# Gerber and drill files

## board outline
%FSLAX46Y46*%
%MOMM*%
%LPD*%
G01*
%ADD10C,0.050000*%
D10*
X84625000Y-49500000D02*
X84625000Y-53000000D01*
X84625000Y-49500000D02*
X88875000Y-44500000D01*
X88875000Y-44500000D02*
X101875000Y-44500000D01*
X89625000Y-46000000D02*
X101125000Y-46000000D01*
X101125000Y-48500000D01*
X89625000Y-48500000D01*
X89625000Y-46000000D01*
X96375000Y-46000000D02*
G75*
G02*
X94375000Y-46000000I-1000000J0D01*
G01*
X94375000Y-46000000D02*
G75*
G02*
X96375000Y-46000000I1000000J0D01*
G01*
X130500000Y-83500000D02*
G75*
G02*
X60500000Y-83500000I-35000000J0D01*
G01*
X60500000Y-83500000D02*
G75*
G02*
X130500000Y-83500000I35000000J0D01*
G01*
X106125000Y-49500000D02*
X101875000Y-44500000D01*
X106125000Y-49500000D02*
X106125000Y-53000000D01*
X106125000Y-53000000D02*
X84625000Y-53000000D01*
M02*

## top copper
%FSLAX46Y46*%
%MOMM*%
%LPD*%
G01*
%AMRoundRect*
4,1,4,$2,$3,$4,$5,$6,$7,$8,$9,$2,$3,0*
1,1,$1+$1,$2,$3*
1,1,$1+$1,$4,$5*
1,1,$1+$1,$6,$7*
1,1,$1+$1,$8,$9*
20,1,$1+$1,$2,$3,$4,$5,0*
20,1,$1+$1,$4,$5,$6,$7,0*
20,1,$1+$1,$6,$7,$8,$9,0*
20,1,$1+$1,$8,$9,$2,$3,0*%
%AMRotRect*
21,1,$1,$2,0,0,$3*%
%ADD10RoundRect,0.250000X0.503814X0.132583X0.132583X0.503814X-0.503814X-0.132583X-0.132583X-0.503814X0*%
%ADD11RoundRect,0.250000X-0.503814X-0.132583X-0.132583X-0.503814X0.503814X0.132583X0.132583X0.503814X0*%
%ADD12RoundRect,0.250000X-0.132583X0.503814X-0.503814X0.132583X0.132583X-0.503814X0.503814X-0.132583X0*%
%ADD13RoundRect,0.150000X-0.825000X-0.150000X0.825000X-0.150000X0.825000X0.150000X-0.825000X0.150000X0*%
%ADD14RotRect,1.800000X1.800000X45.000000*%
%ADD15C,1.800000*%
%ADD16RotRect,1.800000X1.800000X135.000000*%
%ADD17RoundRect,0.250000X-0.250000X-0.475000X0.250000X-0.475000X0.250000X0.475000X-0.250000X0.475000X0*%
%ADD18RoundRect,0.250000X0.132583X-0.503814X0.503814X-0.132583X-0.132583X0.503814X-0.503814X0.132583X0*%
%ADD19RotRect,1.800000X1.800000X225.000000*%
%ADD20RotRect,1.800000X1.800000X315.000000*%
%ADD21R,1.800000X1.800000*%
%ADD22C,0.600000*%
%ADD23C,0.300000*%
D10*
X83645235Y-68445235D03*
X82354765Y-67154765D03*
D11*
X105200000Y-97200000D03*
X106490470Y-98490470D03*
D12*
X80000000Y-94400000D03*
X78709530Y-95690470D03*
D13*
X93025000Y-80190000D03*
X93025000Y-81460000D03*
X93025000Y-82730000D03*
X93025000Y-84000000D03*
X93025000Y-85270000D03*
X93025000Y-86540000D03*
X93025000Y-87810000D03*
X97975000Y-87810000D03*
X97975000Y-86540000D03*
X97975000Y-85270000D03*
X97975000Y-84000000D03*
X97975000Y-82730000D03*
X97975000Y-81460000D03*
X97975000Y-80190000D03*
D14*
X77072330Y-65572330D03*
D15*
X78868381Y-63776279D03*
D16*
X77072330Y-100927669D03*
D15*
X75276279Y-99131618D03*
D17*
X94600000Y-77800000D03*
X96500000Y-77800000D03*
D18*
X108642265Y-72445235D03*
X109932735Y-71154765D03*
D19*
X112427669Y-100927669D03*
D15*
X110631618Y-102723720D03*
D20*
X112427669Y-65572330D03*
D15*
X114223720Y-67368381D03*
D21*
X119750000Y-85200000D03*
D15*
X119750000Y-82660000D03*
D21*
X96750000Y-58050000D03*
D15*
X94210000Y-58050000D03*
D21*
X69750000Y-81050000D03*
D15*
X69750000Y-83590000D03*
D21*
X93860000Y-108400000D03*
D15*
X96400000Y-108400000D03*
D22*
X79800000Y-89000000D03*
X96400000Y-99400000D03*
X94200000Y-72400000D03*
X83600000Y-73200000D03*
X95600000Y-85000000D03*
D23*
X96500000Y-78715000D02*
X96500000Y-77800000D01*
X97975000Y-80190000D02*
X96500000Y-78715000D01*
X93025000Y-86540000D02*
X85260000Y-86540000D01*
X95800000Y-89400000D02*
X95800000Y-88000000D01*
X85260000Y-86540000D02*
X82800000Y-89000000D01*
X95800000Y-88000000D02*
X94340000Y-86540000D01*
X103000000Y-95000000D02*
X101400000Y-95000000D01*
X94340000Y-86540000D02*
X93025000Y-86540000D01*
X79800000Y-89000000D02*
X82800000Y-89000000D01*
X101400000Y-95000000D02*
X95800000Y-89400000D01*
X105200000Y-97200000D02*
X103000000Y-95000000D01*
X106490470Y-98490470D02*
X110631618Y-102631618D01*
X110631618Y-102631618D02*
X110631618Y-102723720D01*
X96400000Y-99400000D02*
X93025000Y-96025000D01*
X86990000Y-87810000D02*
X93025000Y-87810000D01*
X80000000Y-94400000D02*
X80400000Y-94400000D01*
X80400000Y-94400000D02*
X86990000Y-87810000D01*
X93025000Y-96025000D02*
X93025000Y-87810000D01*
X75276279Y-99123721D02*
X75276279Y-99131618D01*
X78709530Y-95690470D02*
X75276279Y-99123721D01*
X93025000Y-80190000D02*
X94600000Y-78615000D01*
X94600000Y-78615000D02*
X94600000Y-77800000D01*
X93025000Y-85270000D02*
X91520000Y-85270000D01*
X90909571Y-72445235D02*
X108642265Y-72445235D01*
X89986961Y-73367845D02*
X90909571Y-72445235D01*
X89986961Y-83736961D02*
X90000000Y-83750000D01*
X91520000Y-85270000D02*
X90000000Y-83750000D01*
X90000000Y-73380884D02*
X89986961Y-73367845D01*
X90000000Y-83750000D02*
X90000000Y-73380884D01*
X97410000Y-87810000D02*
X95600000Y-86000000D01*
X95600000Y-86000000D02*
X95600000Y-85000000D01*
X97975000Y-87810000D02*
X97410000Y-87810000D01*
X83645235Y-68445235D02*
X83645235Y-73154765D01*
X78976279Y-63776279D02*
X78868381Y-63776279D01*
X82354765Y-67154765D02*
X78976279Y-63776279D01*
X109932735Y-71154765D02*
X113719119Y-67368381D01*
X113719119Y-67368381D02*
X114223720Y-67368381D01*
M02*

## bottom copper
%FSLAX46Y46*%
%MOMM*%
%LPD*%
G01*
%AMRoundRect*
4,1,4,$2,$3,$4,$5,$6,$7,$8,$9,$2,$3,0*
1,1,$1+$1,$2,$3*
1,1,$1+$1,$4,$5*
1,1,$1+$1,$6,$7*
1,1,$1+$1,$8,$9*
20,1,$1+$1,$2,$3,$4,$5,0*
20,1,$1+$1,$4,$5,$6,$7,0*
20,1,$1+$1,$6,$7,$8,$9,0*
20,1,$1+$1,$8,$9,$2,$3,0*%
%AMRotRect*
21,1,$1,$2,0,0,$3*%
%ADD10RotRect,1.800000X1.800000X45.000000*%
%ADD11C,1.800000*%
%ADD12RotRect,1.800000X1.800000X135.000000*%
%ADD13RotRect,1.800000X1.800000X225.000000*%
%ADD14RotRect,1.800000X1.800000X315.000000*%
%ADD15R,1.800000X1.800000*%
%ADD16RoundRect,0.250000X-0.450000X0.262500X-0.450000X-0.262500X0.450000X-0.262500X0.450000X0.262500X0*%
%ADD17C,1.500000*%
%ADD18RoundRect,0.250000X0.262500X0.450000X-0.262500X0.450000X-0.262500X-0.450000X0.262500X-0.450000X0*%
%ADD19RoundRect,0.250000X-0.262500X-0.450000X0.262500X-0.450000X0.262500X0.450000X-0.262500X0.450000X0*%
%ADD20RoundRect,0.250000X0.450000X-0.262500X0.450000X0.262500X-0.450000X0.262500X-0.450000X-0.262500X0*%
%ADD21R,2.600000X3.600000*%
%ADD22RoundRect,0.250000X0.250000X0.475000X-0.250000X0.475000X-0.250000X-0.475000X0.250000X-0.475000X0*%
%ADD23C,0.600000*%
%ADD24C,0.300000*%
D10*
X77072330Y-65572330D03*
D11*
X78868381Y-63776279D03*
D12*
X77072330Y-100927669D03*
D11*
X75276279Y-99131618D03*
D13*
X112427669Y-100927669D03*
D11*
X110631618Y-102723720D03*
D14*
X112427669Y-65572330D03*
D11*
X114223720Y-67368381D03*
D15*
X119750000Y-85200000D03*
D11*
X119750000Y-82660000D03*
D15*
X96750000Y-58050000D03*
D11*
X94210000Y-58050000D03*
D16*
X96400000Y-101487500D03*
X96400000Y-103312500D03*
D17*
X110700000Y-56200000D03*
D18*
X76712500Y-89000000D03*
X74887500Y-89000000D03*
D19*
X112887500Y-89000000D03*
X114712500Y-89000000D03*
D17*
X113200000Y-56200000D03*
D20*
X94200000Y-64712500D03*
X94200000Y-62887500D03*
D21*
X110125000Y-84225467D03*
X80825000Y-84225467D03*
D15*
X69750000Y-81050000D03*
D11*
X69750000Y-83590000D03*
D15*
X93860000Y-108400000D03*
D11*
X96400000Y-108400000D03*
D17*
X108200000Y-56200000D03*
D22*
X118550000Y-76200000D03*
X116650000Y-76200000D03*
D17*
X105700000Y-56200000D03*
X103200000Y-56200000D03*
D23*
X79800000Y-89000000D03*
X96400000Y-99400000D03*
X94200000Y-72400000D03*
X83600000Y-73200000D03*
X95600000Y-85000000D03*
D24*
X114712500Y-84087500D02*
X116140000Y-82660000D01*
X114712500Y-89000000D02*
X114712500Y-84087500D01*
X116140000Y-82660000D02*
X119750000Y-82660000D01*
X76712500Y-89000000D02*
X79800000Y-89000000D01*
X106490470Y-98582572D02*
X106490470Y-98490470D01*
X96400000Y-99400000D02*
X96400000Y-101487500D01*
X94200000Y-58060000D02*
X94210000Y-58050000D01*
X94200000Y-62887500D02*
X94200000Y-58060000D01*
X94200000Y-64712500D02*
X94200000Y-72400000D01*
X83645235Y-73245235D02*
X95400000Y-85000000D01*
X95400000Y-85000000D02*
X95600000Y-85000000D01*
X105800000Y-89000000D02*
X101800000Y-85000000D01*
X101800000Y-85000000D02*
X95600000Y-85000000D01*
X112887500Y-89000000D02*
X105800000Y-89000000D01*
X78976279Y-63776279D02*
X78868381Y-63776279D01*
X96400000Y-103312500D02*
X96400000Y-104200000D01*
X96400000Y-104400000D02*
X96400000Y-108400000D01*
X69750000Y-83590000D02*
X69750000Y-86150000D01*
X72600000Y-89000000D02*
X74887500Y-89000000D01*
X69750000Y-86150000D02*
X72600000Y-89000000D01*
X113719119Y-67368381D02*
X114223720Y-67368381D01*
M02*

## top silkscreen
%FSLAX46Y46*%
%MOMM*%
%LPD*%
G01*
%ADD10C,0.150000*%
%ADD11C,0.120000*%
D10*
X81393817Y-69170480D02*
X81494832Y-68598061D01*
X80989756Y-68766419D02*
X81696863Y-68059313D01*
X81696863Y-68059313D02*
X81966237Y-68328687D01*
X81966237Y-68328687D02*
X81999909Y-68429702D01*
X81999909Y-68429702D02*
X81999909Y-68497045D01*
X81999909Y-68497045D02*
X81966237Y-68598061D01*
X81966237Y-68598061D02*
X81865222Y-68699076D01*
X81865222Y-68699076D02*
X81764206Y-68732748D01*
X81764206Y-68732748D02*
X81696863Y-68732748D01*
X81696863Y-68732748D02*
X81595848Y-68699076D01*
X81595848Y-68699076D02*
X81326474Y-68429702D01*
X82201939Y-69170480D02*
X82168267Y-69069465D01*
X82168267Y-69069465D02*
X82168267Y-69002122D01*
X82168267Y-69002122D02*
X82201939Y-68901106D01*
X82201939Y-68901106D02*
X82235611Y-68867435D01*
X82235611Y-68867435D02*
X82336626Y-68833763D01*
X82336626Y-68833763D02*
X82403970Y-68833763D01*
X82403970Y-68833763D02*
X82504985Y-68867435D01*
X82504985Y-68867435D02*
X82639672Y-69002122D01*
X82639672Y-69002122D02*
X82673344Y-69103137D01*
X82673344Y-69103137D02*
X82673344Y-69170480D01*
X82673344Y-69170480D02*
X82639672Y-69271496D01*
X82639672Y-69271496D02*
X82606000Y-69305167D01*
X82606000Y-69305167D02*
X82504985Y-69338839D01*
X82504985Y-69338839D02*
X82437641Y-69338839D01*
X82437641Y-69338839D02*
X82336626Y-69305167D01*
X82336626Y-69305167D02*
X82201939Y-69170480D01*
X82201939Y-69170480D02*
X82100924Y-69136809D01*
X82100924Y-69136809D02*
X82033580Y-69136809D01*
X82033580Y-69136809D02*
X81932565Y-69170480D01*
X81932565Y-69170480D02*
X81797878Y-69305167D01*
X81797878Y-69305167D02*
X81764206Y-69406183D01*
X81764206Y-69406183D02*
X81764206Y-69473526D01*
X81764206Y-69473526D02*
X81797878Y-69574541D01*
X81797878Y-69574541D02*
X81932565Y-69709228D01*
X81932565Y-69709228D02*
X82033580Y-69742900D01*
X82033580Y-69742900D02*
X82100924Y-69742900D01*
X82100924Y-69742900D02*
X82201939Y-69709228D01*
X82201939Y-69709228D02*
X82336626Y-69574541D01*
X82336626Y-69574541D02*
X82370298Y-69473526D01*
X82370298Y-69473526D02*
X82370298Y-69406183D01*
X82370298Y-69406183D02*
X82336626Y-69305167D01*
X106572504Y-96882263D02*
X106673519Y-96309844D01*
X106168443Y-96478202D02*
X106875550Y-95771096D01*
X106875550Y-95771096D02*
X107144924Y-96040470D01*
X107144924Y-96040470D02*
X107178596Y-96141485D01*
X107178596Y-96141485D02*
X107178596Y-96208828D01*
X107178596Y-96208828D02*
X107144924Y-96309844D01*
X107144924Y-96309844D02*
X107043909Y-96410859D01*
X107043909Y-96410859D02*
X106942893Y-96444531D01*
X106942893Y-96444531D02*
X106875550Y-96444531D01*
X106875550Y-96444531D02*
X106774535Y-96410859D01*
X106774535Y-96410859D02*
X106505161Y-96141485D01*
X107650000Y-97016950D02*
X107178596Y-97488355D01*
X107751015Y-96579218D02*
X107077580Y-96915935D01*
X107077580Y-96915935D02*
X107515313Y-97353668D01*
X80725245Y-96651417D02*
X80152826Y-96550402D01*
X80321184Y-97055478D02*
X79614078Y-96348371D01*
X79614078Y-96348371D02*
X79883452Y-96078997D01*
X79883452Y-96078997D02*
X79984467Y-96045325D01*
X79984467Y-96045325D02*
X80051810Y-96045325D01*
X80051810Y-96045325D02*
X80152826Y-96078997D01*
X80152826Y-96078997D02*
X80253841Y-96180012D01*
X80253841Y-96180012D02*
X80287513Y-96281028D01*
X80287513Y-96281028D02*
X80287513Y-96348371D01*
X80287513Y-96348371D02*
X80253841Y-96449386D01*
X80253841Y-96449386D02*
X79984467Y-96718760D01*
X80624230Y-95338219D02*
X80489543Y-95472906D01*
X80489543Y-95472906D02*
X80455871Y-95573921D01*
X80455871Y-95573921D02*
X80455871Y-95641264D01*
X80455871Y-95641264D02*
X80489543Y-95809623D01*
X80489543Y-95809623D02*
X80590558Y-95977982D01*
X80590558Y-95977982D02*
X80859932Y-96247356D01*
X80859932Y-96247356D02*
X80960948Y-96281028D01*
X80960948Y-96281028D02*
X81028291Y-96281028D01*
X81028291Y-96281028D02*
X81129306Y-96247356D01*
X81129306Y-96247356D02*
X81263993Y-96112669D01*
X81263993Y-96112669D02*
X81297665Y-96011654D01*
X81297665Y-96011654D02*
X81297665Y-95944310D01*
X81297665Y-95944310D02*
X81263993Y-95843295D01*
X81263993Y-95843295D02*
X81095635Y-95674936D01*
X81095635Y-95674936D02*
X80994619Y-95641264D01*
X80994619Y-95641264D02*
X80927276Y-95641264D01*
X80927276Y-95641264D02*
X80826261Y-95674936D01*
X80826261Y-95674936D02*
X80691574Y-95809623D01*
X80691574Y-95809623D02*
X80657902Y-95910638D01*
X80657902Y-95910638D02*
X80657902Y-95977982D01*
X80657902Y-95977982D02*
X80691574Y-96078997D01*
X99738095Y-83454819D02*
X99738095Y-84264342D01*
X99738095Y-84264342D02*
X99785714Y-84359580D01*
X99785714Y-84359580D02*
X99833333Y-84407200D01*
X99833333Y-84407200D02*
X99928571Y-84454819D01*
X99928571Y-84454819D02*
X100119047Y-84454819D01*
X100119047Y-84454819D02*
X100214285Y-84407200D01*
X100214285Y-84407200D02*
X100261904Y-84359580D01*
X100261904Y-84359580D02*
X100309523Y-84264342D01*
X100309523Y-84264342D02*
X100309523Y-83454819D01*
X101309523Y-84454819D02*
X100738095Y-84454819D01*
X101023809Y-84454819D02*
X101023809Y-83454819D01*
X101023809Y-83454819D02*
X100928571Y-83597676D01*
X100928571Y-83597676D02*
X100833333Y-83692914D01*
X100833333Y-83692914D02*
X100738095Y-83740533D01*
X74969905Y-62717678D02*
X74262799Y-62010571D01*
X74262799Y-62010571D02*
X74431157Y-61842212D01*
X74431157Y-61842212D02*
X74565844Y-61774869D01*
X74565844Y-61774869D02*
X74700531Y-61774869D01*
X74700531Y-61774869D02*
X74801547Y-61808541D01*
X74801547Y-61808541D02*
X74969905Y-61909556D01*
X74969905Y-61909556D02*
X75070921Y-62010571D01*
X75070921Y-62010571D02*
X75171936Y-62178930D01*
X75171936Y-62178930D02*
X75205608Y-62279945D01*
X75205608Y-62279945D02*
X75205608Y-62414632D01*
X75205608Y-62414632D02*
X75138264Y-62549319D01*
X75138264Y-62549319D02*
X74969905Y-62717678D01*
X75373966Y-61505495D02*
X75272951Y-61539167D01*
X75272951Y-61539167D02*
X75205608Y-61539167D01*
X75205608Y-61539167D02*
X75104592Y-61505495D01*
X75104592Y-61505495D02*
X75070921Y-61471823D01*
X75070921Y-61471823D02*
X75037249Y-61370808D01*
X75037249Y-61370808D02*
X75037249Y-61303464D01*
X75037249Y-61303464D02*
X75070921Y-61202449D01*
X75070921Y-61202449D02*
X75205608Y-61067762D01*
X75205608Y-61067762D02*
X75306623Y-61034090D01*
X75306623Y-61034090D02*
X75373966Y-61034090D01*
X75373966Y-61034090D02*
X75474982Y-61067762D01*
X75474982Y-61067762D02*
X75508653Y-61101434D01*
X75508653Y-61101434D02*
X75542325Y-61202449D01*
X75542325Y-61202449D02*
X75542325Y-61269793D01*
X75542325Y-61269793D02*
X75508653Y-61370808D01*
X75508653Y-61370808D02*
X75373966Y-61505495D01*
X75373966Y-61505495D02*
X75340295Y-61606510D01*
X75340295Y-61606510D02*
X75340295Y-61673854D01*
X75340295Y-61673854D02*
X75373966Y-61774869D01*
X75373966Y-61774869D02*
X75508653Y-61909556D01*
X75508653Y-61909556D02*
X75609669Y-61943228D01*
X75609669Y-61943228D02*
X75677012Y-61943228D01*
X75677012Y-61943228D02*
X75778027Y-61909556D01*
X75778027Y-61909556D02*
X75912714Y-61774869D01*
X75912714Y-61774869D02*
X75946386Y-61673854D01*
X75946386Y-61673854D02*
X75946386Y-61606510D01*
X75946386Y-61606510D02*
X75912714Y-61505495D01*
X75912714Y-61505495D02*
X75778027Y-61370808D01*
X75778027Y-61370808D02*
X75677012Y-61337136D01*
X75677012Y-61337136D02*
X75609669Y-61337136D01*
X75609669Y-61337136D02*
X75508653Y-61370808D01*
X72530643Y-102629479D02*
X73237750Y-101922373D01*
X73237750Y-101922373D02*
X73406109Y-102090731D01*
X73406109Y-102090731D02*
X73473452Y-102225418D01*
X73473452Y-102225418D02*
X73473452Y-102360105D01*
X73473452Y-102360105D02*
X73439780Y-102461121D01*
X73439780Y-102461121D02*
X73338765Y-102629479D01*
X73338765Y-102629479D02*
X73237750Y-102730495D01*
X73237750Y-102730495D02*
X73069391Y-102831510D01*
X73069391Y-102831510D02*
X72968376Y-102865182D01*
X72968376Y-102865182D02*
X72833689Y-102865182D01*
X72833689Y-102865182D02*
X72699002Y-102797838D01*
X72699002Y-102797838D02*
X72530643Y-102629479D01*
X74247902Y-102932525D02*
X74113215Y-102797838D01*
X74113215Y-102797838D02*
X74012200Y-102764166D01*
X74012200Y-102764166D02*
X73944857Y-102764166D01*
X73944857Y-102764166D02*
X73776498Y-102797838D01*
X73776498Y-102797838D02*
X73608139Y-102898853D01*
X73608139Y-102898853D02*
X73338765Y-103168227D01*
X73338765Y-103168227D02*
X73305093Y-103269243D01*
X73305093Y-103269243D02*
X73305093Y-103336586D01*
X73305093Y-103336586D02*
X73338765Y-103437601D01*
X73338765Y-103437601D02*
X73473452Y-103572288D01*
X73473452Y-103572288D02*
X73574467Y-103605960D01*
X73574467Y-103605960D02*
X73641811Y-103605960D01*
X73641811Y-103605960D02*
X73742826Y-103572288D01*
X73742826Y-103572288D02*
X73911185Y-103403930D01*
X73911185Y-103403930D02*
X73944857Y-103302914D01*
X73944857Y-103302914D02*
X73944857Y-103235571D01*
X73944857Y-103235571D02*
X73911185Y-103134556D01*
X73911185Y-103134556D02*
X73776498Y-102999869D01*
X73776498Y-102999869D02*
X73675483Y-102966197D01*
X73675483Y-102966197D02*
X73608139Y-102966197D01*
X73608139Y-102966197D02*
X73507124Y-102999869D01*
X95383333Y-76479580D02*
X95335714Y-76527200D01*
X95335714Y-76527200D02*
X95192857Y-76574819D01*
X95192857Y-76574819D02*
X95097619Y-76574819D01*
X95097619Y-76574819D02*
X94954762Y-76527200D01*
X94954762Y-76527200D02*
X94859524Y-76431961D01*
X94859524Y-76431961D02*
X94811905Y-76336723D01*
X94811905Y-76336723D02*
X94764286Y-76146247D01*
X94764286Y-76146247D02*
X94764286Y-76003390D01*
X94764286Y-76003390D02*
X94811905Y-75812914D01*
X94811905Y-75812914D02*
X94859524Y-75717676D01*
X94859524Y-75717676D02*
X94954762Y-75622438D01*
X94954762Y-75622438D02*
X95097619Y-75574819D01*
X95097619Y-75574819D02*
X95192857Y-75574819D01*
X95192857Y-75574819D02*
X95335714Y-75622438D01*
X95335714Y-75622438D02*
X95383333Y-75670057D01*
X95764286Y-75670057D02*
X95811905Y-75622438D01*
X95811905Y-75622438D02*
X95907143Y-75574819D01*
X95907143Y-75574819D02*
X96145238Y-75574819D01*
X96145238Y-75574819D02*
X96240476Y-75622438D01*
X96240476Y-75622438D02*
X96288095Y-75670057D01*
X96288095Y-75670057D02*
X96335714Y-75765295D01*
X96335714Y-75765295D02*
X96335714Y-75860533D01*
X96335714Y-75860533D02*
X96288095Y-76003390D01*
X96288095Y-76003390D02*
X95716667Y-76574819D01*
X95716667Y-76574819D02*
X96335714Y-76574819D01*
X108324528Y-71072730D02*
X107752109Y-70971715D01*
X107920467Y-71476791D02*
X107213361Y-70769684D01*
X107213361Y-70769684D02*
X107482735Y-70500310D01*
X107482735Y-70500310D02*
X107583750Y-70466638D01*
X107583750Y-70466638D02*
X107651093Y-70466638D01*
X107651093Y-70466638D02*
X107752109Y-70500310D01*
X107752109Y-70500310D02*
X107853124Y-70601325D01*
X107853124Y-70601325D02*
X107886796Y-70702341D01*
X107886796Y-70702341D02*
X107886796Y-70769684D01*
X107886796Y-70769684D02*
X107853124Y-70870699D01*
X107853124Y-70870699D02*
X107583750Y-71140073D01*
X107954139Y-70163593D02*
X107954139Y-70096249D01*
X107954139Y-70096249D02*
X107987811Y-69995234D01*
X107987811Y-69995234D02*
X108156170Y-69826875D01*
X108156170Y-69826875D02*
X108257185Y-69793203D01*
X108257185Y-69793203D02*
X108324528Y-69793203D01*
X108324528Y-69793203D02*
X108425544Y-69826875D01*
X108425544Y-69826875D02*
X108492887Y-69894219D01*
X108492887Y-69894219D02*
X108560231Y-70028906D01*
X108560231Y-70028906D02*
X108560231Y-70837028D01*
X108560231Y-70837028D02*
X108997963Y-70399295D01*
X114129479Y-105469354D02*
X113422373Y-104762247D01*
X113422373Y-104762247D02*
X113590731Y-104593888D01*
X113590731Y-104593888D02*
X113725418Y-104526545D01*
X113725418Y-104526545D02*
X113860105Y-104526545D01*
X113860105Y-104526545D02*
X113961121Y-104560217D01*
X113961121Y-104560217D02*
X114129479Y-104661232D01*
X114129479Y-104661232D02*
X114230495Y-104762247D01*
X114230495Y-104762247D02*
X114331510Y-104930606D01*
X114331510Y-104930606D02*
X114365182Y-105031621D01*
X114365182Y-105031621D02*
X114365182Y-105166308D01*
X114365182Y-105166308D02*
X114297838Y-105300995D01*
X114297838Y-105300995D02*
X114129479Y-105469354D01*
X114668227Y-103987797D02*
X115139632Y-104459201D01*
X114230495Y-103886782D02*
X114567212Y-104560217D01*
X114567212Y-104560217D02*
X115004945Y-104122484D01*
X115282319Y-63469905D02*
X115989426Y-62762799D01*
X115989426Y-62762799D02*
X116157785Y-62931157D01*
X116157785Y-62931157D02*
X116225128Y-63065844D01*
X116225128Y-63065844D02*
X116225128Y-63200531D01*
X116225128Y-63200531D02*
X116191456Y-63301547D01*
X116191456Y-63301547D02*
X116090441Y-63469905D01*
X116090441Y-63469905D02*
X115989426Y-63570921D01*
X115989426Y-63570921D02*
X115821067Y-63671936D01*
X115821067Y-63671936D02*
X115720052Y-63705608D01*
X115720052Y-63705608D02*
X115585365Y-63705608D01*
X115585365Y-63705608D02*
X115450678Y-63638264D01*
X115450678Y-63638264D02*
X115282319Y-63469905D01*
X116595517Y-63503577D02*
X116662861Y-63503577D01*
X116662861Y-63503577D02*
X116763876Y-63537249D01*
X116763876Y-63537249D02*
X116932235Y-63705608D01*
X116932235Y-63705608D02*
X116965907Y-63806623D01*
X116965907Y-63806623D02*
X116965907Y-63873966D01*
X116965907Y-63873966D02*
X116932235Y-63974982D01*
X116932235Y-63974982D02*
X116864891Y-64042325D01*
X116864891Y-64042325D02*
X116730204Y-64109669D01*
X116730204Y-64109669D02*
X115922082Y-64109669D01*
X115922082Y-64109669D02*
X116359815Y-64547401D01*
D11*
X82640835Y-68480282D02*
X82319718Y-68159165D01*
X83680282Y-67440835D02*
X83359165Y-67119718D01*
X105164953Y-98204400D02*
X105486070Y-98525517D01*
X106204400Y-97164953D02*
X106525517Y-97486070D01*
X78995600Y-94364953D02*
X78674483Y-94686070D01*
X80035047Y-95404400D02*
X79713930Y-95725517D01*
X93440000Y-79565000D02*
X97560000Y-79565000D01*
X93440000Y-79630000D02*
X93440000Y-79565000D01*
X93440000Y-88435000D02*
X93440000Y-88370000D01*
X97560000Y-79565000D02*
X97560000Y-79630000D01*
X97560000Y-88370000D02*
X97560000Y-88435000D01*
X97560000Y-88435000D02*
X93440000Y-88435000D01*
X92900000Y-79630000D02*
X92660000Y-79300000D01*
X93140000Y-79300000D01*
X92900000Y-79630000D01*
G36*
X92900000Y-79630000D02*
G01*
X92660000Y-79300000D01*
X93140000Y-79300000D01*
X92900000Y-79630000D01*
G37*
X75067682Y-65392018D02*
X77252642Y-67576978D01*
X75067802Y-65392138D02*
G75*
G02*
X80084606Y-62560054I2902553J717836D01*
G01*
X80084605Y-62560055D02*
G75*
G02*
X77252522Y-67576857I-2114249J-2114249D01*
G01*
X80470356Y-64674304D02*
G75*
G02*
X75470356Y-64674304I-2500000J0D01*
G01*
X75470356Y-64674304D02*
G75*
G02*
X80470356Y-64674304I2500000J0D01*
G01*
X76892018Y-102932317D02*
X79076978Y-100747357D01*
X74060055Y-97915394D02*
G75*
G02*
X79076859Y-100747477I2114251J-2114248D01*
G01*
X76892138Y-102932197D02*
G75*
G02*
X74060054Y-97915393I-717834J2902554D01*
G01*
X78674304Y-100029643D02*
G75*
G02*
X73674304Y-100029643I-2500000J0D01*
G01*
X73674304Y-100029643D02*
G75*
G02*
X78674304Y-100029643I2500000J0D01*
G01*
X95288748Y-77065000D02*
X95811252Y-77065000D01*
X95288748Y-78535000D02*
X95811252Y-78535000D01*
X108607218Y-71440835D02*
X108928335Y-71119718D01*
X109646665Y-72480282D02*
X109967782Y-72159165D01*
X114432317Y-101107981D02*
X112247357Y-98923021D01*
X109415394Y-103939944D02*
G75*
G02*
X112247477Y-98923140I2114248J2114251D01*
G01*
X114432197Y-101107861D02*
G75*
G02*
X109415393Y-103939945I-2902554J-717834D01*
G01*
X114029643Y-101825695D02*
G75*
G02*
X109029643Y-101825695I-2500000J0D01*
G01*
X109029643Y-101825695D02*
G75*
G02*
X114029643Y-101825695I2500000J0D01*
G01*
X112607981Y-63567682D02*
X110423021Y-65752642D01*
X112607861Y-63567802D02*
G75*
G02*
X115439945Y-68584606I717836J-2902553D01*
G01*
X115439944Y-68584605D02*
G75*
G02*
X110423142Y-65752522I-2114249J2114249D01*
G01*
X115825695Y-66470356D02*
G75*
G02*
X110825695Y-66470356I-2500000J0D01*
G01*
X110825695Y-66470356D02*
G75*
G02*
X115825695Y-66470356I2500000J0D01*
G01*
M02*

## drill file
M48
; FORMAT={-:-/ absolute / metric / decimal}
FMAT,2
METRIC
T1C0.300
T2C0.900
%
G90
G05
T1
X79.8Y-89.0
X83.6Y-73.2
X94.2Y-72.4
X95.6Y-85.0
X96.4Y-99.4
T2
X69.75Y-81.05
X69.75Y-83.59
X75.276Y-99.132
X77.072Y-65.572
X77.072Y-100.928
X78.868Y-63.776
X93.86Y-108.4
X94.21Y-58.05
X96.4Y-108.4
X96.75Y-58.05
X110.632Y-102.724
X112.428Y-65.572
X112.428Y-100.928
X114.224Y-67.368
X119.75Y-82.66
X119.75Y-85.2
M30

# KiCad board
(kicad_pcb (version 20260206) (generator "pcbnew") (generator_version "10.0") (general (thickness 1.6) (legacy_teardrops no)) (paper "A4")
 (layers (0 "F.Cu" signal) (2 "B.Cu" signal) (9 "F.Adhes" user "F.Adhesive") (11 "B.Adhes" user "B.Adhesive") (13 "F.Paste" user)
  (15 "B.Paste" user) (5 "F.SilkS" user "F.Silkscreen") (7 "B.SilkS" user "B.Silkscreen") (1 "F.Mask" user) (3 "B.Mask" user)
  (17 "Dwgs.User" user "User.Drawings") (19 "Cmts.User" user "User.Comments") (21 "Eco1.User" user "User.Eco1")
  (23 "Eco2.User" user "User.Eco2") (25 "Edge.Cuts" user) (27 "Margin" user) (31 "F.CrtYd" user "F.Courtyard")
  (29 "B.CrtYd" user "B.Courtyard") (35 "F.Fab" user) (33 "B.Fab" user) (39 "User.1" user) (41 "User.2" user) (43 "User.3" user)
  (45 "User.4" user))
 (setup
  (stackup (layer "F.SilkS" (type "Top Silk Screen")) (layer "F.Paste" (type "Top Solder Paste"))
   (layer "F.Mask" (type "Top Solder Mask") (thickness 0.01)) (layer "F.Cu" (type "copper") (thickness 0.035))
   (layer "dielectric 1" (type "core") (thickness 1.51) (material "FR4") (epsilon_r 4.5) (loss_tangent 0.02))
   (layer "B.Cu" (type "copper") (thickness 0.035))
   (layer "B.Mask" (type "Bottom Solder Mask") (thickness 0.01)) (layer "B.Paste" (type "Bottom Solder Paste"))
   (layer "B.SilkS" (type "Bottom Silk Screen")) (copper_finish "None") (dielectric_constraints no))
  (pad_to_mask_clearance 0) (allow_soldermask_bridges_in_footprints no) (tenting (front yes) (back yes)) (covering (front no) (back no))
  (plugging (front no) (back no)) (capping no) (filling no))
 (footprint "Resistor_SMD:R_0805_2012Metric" (layer "F.Cu") (at 83 67.8 135)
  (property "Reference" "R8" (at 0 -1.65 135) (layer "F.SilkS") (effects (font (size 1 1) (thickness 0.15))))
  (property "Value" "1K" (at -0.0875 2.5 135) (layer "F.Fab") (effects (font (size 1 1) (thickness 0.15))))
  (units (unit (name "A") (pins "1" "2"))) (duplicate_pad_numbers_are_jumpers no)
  (fp_line (start -0.227064 -0.735) (end 0.227064 -0.735) (stroke (width 0.12) (type solid)) (layer "F.SilkS"))
  (fp_line (start -0.227064 0.735) (end 0.227064 0.735) (stroke (width 0.12) (type solid)) (layer "F.SilkS"))
  (pad "1" smd roundrect (at -0.9125 0 135) (size 1.025 1.4) (layers "F.Cu" "F.Mask" "F.Paste") (roundrect_rratio 0.243902)
   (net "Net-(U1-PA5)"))
  (pad "2" smd roundrect (at 0.9125 0 135) (size 1.025 1.4) (layers "F.Cu" "F.Mask" "F.Paste") (roundrect_rratio 0.243902)
   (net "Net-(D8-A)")))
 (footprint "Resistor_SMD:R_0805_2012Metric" (layer "F.Cu") (at 105.845235 97.845235 -45)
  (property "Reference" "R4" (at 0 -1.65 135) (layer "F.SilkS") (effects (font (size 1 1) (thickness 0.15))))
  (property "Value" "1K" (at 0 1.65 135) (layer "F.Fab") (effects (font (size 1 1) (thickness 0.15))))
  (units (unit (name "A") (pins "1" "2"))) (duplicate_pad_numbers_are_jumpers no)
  (fp_line (start -0.227064 0.735) (end 0.227064 0.735) (stroke (width 0.12) (type solid)) (layer "F.SilkS"))
  (fp_line (start -0.227064 -0.735) (end 0.227064 -0.735) (stroke (width 0.12) (type solid)) (layer "F.SilkS"))
  (pad "1" smd roundrect (at -0.9125 0 315) (size 1.025 1.4) (layers "F.Cu" "F.Mask" "F.Paste") (roundrect_rratio 0.243902)
   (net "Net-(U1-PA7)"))
  (pad "2" smd roundrect (at 0.9125 0 315) (size 1.025 1.4) (layers "F.Cu" "F.Mask" "F.Paste") (roundrect_rratio 0.243902)
   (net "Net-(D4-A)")))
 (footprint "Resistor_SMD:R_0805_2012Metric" (layer "F.Cu") (at 79.354765 95.045235 -135)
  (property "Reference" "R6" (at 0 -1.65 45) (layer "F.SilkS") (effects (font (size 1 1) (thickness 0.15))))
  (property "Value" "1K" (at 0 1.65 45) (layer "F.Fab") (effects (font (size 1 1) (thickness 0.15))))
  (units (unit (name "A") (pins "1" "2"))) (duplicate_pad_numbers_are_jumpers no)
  (fp_line (start -0.227064 0.735) (end 0.227064 0.735) (stroke (width 0.12) (type solid)) (layer "F.SilkS"))
  (fp_line (start -0.227064 -0.735) (end 0.227064 -0.735) (stroke (width 0.12) (type solid)) (layer "F.SilkS"))
  (pad "1" smd roundrect (at -0.9125 0 225) (size 1.025 1.4) (layers "F.Cu" "F.Mask" "F.Paste") (roundrect_rratio 0.243902)
   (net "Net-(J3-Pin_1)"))
  (pad "2" smd roundrect (at 0.9125 0 225) (size 1.025 1.4) (layers "F.Cu" "F.Mask" "F.Paste") (roundrect_rratio 0.243902)
   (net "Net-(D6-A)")))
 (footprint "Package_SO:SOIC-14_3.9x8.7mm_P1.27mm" (layer "F.Cu") (at 95.5 84)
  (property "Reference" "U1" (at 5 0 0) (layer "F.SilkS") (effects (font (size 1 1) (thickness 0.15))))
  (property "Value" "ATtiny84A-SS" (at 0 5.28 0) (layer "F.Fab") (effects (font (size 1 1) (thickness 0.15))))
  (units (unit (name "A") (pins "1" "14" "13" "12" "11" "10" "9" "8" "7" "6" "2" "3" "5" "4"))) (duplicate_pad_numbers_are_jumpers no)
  (fp_line (start -2.06 -4.435) (end 2.06 -4.435) (stroke (width 0.12) (type solid)) (layer "F.SilkS"))
  (fp_line (start -2.06 -4.37) (end -2.06 -4.435) (stroke (width 0.12) (type solid)) (layer "F.SilkS"))
  (fp_line (start -2.06 4.435) (end -2.06 4.37) (stroke (width 0.12) (type solid)) (layer "F.SilkS"))
  (fp_line (start 2.06 -4.435) (end 2.06 -4.37) (stroke (width 0.12) (type solid)) (layer "F.SilkS"))
  (fp_line (start 2.06 4.37) (end 2.06 4.435) (stroke (width 0.12) (type solid)) (layer "F.SilkS"))
  (fp_line (start 2.06 4.435) (end -2.06 4.435) (stroke (width 0.12) (type solid)) (layer "F.SilkS"))
  (fp_poly (pts (xy -2.6 -4.37) (xy -2.84 -4.7) (xy -2.36 -4.7)) (stroke (width 0.12) (type solid)) (fill yes) (layer "F.SilkS"))
  (pad "1" smd roundrect (at -2.475 -3.81) (size 1.95 0.6) (layers "F.Cu" "F.Mask" "F.Paste") (roundrect_rratio 0.25) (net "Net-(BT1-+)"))
  (pad "2" smd roundrect (at -2.475 -2.54) (size 1.95 0.6) (layers "F.Cu" "F.Mask" "F.Paste") (roundrect_rratio 0.25)
   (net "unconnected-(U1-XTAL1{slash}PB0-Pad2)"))
  (pad "3" smd roundrect (at -2.475 -1.27) (size 1.95 0.6) (layers "F.Cu" "F.Mask" "F.Paste") (roundrect_rratio 0.25)
   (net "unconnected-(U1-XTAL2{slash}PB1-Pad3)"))
  (pad "4" smd roundrect (at -2.475 0) (size 1.95 0.6) (layers "F.Cu" "F.Mask" "F.Paste") (roundrect_rratio 0.25) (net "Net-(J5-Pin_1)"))
  (pad "5" smd roundrect (at -2.475 1.27) (size 1.95 0.6) (layers "F.Cu" "F.Mask" "F.Paste") (roundrect_rratio 0.25) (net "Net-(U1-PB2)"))
  (pad "6" smd roundrect (at -2.475 2.54) (size 1.95 0.6) (layers "F.Cu" "F.Mask" "F.Paste") (roundrect_rratio 0.25) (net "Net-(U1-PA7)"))
  (pad "7" smd roundrect (at -2.475 3.81) (size 1.95 0.6) (layers "F.Cu" "F.Mask" "F.Paste") (roundrect_rratio 0.25) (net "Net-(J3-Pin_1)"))
  (pad "8" smd roundrect (at 2.475 3.81) (size 1.95 0.6) (layers "F.Cu" "F.Mask" "F.Paste") (roundrect_rratio 0.25) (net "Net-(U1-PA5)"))
  (pad "9" smd roundrect (at 2.475 2.54) (size 1.95 0.6) (layers "F.Cu" "F.Mask" "F.Paste") (roundrect_rratio 0.25) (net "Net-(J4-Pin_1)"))
  (pad "10" smd roundrect (at 2.475 1.27) (size 1.95 0.6) (layers "F.Cu" "F.Mask" "F.Paste") (roundrect_rratio 0.25)
   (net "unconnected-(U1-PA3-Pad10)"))
  (pad "11" smd roundrect (at 2.475 0) (size 1.95 0.6) (layers "F.Cu" "F.Mask" "F.Paste") (roundrect_rratio 0.25)
   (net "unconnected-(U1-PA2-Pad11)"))
  (pad "12" smd roundrect (at 2.475 -1.27) (size 1.95 0.6) (layers "F.Cu" "F.Mask" "F.Paste") (roundrect_rratio 0.25) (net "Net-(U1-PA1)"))
  (pad "13" smd roundrect (at 2.475 -2.54) (size 1.95 0.6) (layers "F.Cu" "F.Mask" "F.Paste") (roundrect_rratio 0.25)
   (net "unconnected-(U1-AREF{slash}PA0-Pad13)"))
  (pad "14" smd roundrect (at 2.475 -3.81) (size 1.95 0.6) (layers "F.Cu" "F.Mask" "F.Paste") (roundrect_rratio 0.25) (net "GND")))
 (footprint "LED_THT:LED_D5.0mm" (layer "F.Cu") (at 77.07233 65.57233 45)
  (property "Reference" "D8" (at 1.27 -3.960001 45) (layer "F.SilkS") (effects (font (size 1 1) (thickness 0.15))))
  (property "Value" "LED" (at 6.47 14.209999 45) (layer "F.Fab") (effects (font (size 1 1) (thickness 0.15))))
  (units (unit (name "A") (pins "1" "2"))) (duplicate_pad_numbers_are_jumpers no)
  (fp_line (start -1.29 -1.545) (end -1.29 1.545) (stroke (width 0.12) (type solid)) (layer "F.SilkS"))
  (fp_arc (start -1.29 -1.54483) (mid 2.07178 -2.880496) (end 4.26 0) (stroke (width 0.12) (type solid)) (layer "F.SilkS"))
  (fp_arc (start 4.26 0) (mid 2.07178 2.880495) (end -1.29 1.54483) (stroke (width 0.12) (type solid)) (layer "F.SilkS"))
  (fp_circle (center 1.270001 0) (end 3.770001 0) (stroke (width 0.12) (type solid)) (fill no) (layer "F.SilkS"))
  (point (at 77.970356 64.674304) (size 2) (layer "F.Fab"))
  (pad "1" thru_hole rect (at 0 0 45) (size 1.8 1.8) (drill 0.9) (layers "*.Cu" "*.Mask") (remove_unused_layers no) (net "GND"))
  (pad "2" thru_hole circle (at 2.54 0 45) (size 1.8 1.8) (drill 0.9) (layers "*.Cu" "*.Mask") (remove_unused_layers no) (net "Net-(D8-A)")))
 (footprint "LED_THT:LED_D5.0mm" (layer "F.Cu") (at 77.07233 100.927669 135)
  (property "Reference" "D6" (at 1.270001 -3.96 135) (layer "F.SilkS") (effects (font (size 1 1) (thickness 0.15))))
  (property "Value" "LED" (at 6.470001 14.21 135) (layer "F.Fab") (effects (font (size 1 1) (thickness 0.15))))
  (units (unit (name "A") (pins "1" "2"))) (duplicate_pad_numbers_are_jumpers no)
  (fp_line (start -1.29 -1.545) (end -1.29 1.545) (stroke (width 0.12) (type solid)) (layer "F.SilkS"))
  (fp_arc (start 4.26 0) (mid 2.071779 2.880496) (end -1.29 1.54483) (stroke (width 0.12) (type solid)) (layer "F.SilkS"))
  (fp_arc (start -1.29 -1.54483) (mid 2.071779 -2.880496) (end 4.26 0) (stroke (width 0.12) (type solid)) (layer "F.SilkS"))
  (fp_circle (center 1.270001 0) (end 3.770001 0) (stroke (width 0.12) (type solid)) (fill no) (layer "F.SilkS"))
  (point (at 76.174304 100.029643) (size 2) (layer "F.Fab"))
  (pad "1" thru_hole rect (at 0 0 135) (size 1.8 1.8) (drill 0.9) (layers "*.Cu" "*.Mask") (remove_unused_layers no) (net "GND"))
  (pad "2" thru_hole circle (at 2.54 0 135) (size 1.8 1.8) (drill 0.9) (layers "*.Cu" "*.Mask") (remove_unused_layers no) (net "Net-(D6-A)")))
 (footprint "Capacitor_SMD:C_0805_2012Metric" (layer "F.Cu") (at 95.55 77.8)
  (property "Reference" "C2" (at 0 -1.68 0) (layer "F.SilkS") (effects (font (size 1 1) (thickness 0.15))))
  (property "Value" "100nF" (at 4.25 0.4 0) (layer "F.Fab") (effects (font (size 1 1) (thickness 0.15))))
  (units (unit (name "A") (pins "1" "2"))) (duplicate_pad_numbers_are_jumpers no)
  (fp_line (start -0.261252 -0.735) (end 0.261252 -0.735) (stroke (width 0.12) (type solid)) (layer "F.SilkS"))
  (fp_line (start -0.261252 0.735) (end 0.261252 0.735) (stroke (width 0.12) (type solid)) (layer "F.SilkS"))
  (pad "1" smd roundrect (at -0.95 0) (size 1 1.45) (layers "F.Cu" "F.Mask" "F.Paste") (roundrect_rratio 0.25) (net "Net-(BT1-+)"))
  (pad "2" smd roundrect (at 0.95 0) (size 1 1.45) (layers "F.Cu" "F.Mask" "F.Paste") (roundrect_rratio 0.25) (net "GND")))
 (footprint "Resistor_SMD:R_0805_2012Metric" (layer "F.Cu") (at 109.2875 71.8 45)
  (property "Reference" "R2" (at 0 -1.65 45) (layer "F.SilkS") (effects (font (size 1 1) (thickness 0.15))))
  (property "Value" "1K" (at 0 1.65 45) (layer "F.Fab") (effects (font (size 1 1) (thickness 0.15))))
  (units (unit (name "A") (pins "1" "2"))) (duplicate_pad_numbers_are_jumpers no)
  (fp_line (start -0.227064 -0.735) (end 0.227064 -0.735) (stroke (width 0.12) (type solid)) (layer "F.SilkS"))
  (fp_line (start -0.227064 0.735) (end 0.227064 0.735) (stroke (width 0.12) (type solid)) (layer "F.SilkS"))
  (pad "1" smd roundrect (at -0.9125 0 45) (size 1.025 1.4) (layers "F.Cu" "F.Mask" "F.Paste") (roundrect_rratio 0.243902)
   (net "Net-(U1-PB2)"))
  (pad "2" smd roundrect (at 0.9125 0 45) (size 1.025 1.4) (layers "F.Cu" "F.Mask" "F.Paste") (roundrect_rratio 0.243902) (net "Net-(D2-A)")))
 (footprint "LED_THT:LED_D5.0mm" (layer "F.Cu") (at 112.427669 100.927669 -135)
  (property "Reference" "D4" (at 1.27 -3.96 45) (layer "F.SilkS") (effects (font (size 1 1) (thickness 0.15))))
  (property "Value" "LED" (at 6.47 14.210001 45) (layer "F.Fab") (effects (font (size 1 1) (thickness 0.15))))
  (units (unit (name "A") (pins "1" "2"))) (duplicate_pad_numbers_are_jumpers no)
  (fp_line (start -1.29 -1.545) (end -1.29 1.545) (stroke (width 0.12) (type solid)) (layer "F.SilkS"))
  (fp_arc (start 4.26 0) (mid 2.071779 2.880496) (end -1.29 1.54483) (stroke (width 0.12) (type solid)) (layer "F.SilkS"))
  (fp_arc (start -1.29 -1.54483) (mid 2.071779 -2.880496) (end 4.26 0) (stroke (width 0.12) (type solid)) (layer "F.SilkS"))
  (fp_circle (center 1.270001 0) (end 3.770001 0) (stroke (width 0.12) (type solid)) (fill no) (layer "F.SilkS"))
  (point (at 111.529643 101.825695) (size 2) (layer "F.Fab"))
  (pad "1" thru_hole rect (at 0 0 225) (size 1.8 1.8) (drill 0.9) (layers "*.Cu" "*.Mask") (remove_unused_layers no) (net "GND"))
  (pad "2" thru_hole circle (at 2.54 0 225) (size 1.8 1.8) (drill 0.9) (layers "*.Cu" "*.Mask") (remove_unused_layers no) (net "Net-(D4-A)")))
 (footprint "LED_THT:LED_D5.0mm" (layer "F.Cu") (at 112.427669 65.57233 -45)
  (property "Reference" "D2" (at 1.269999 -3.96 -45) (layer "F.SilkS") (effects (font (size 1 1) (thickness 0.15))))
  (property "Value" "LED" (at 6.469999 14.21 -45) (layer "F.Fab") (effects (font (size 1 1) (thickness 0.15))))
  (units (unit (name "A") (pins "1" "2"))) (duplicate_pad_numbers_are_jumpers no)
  (fp_line (start -1.29 -1.545) (end -1.29 1.545) (stroke (width 0.12) (type solid)) (layer "F.SilkS"))
  (fp_arc (start -1.29 -1.54483) (mid 2.07178 -2.880496) (end 4.26 0) (stroke (width 0.12) (type solid)) (layer "F.SilkS"))
  (fp_arc (start 4.26 0) (mid 2.07178 2.880495) (end -1.29 1.54483) (stroke (width 0.12) (type solid)) (layer "F.SilkS"))
  (fp_circle (center 1.270001 0) (end 3.770001 0) (stroke (width 0.12) (type solid)) (fill no) (layer "F.SilkS"))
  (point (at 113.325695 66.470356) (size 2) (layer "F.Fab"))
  (pad "1" thru_hole rect (at 0 0 315) (size 1.8 1.8) (drill 0.9) (layers "*.Cu" "*.Mask") (remove_unused_layers no) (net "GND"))
  (pad "2" thru_hole circle (at 2.54 0 315) (size 1.8 1.8) (drill 0.9) (layers "*.Cu" "*.Mask") (remove_unused_layers no) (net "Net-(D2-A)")))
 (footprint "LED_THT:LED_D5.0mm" (layer "B.Cu") (at 119.75 85.2 90)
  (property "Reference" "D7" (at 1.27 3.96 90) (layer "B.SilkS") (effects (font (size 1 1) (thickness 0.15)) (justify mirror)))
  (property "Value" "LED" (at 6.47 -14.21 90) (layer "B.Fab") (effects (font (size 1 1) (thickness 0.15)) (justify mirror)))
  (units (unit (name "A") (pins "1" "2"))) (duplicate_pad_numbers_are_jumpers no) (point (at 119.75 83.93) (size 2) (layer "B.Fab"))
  (pad "1" thru_hole rect (at 0 0 90) (size 1.8 1.8) (drill 0.9) (layers "*.Cu" "*.Mask") (remove_unused_layers no) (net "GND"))
  (pad "2" thru_hole circle (at 2.54 0 90) (size 1.8 1.8) (drill 0.9) (layers "*.Cu" "*.Mask") (remove_unused_layers no) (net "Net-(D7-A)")))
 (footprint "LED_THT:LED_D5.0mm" (layer "B.Cu") (at 96.75 58.05 180)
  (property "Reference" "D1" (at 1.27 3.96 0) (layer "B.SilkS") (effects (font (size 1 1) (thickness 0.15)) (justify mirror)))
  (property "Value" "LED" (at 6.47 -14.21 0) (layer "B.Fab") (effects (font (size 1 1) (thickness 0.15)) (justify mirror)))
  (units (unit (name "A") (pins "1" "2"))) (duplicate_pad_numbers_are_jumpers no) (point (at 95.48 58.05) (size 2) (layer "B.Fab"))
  (pad "1" thru_hole rect (at 0 0 180) (size 1.8 1.8) (drill 0.9) (layers "*.Cu" "*.Mask") (remove_unused_layers no) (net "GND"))
  (pad "2" thru_hole circle (at 2.54 0 180) (size 1.8 1.8) (drill 0.9) (layers "*.Cu" "*.Mask") (remove_unused_layers no) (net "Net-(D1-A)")))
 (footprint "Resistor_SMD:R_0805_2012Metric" (layer "B.Cu") (at 96.4 102.4 -90)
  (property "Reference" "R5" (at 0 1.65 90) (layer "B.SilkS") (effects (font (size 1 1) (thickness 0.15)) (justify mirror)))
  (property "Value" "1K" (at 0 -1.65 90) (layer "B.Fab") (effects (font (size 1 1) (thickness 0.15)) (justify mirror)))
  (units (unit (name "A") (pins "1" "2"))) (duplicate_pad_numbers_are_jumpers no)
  (pad "1" smd roundrect (at -0.9125 0 270) (size 1.025 1.4) (layers "B.Cu" "B.Mask" "B.Paste") (roundrect_rratio 0.243902)
   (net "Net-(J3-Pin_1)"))
  (pad "2" smd roundrect (at 0.9125 0 270) (size 1.025 1.4) (layers "B.Cu" "B.Mask" "B.Paste") (roundrect_rratio 0.243902)
   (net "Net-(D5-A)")))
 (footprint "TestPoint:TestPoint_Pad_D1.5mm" (layer "B.Cu") (at 110.7 56.2 180)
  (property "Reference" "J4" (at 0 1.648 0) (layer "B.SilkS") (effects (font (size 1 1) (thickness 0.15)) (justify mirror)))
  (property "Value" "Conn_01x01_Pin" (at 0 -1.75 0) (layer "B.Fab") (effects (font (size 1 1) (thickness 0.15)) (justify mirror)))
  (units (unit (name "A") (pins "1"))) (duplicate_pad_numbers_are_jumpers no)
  (pad "1" smd circle (at 0 0 180) (size 1.5 1.5) (layers "B.Cu" "B.Mask") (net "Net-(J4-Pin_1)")))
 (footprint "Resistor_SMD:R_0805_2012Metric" (layer "B.Cu") (at 75.8 89 180)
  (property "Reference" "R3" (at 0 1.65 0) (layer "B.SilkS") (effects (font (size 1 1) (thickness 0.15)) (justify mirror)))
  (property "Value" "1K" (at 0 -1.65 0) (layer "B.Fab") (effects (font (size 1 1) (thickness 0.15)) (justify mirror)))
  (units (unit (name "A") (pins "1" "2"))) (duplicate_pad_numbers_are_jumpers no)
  (pad "1" smd roundrect (at -0.9125 0 180) (size 1.025 1.4) (layers "B.Cu" "B.Mask" "B.Paste") (roundrect_rratio 0.243902)
   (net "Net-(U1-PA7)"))
  (pad "2" smd roundrect (at 0.9125 0 180) (size 1.025 1.4) (layers "B.Cu" "B.Mask" "B.Paste") (roundrect_rratio 0.243902)
   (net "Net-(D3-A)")))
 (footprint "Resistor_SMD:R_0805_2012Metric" (layer "B.Cu") (at 113.8 89)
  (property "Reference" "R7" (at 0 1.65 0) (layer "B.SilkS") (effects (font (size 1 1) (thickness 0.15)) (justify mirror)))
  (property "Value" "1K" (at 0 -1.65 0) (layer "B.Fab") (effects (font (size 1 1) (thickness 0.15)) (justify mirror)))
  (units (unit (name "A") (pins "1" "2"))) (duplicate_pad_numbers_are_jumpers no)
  (pad "1" smd roundrect (at -0.9125 0) (size 1.025 1.4) (layers "B.Cu" "B.Mask" "B.Paste") (roundrect_rratio 0.243902) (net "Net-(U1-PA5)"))
  (pad "2" smd roundrect (at 0.9125 0) (size 1.025 1.4) (layers "B.Cu" "B.Mask" "B.Paste") (roundrect_rratio 0.243902) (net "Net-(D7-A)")))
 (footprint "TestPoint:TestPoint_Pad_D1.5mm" (layer "B.Cu") (at 113.2 56.2 180)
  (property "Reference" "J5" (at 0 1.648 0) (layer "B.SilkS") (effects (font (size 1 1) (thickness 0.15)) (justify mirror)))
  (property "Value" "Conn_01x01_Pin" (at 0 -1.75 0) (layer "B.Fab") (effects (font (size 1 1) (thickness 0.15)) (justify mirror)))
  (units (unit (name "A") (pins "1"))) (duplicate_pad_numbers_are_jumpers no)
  (pad "1" smd circle (at 0 0 180) (size 1.5 1.5) (layers "B.Cu" "B.Mask") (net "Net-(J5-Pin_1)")))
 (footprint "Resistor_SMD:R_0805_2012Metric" (layer "B.Cu") (at 94.2 63.8 90)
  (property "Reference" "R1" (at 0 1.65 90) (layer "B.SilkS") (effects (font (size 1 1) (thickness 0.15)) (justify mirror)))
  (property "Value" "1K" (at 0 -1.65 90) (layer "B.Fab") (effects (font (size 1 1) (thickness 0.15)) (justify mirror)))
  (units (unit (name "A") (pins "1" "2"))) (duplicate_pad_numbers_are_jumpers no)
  (pad "1" smd roundrect (at -0.9125 0 90) (size 1.025 1.4) (layers "B.Cu" "B.Mask" "B.Paste") (roundrect_rratio 0.243902)
   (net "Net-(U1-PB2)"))
  (pad "2" smd roundrect (at 0.9125 0 90) (size 1.025 1.4) (layers "B.Cu" "B.Mask" "B.Paste") (roundrect_rratio 0.243902) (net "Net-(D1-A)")))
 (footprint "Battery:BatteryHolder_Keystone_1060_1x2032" (layer "B.Cu") (at 95.475 84.225467 180)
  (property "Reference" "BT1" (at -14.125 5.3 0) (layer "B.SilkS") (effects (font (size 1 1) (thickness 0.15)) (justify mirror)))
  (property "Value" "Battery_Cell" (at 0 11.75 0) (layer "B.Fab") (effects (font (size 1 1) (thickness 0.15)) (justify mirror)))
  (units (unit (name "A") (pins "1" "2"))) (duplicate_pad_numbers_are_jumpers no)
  (pad "1" smd rect (at -14.65 0) (size 2.6 3.6) (layers "B.Cu" "B.Mask" "B.Paste") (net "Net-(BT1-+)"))
  (pad "2" smd rect (at 14.65 0) (size 2.6 3.6) (layers "B.Cu" "B.Mask" "B.Paste") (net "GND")))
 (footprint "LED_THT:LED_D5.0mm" (layer "B.Cu") (at 69.75 81.05 -90)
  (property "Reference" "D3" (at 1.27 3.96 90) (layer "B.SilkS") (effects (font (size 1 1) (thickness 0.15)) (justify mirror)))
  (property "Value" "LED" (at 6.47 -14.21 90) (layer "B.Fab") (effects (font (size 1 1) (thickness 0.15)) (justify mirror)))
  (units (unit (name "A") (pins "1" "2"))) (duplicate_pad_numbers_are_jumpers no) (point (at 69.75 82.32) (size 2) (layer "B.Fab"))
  (pad "1" thru_hole rect (at 0 0 270) (size 1.8 1.8) (drill 0.9) (layers "*.Cu" "*.Mask") (remove_unused_layers no) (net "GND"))
  (pad "2" thru_hole circle (at 2.54 0 270) (size 1.8 1.8) (drill 0.9) (layers "*.Cu" "*.Mask") (remove_unused_layers no) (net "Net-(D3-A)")))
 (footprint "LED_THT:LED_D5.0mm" (layer "B.Cu") (at 93.86 108.4)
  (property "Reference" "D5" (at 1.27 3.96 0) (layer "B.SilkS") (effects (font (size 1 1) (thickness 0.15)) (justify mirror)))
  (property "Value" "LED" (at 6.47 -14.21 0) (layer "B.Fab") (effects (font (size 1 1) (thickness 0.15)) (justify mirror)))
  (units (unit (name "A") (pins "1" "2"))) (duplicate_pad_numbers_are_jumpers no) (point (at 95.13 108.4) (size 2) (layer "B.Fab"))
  (pad "1" thru_hole rect (at 0 0) (size 1.8 1.8) (drill 0.9) (layers "*.Cu" "*.Mask") (remove_unused_layers no) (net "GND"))
  (pad "2" thru_hole circle (at 2.54 0) (size 1.8 1.8) (drill 0.9) (layers "*.Cu" "*.Mask") (remove_unused_layers no) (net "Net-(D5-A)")))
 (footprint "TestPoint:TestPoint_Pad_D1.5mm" (layer "B.Cu") (at 108.2 56.2 180)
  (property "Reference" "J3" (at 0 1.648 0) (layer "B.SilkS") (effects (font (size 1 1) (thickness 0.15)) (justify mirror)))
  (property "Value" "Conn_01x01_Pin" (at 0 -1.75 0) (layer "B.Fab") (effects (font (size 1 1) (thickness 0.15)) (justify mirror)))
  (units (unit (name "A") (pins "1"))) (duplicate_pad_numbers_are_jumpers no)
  (pad "1" smd circle (at 0 0 180) (size 1.5 1.5) (layers "B.Cu" "B.Mask") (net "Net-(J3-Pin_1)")))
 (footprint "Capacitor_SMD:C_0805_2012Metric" (layer "B.Cu") (at 117.6 76.2 180)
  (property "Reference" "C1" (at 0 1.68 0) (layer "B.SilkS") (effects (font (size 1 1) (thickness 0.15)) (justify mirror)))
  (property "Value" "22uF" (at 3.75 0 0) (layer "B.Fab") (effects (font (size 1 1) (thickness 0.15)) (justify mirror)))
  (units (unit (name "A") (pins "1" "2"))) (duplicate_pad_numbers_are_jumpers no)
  (pad "1" smd roundrect (at -0.95 0 180) (size 1 1.45) (layers "B.Cu" "B.Mask" "B.Paste") (roundrect_rratio 0.25) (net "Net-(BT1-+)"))
  (pad "2" smd roundrect (at 0.95 0 180) (size 1 1.45) (layers "B.Cu" "B.Mask" "B.Paste") (roundrect_rratio 0.25) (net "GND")))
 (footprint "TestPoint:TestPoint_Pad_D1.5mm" (layer "B.Cu") (at 105.7 56.2 180)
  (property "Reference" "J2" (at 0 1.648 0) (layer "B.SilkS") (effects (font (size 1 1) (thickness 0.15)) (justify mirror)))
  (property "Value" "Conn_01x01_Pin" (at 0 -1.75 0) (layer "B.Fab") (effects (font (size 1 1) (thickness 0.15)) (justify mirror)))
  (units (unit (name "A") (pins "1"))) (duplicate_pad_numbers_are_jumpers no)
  (pad "1" smd circle (at 0 0 180) (size 1.5 1.5) (layers "B.Cu" "B.Mask") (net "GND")))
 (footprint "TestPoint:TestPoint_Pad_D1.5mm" (layer "B.Cu") (at 103.2 56.2 180)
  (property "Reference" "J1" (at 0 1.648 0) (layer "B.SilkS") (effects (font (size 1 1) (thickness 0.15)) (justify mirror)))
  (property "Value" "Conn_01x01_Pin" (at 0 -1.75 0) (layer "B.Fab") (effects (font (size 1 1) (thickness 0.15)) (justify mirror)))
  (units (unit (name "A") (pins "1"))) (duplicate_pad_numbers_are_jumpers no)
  (pad "1" smd circle (at 0 0 180) (size 1.5 1.5) (layers "B.Cu" "B.Mask") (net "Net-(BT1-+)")))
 (gr_line (start 84.625 49.5) (end 84.625 53) (stroke (width 0.05) (type default)) (layer "Edge.Cuts"))
 (gr_line (start 84.625 49.5) (end 88.875 44.5) (stroke (width 0.05) (type default)) (layer "Edge.Cuts"))
 (gr_line (start 88.875 44.5) (end 101.875 44.5) (stroke (width 0.05) (type default)) (layer "Edge.Cuts"))
 (gr_rect (start 89.625 46) (end 101.125 48.5) (stroke (width 0.05) (type default)) (fill no) (layer "Edge.Cuts"))
 (gr_circle (center 95.375 46) (end 96.375 46) (stroke (width 0.05) (type solid)) (fill no) (layer "Edge.Cuts"))
 (gr_circle (center 95.5 83.5) (end 130.5 83.5) (stroke (width 0.05) (type default)) (fill no) (layer "Edge.Cuts"))
 (gr_line (start 106.125 49.5) (end 101.875 44.5) (stroke (width 0.05) (type default)) (layer "Edge.Cuts"))
 (gr_line (start 106.125 49.5) (end 106.125 53) (stroke (width 0.05) (type default)) (layer "Edge.Cuts"))
 (gr_line (start 106.125 53) (end 84.625 53) (stroke (width 0.05) (type default)) (layer "Edge.Cuts"))
 (segment (start 96.5 78.715) (end 96.5 77.8) (width 0.3) (layer "F.Cu") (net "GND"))
 (segment (start 97.975 80.19) (end 96.5 78.715) (width 0.3) (layer "F.Cu") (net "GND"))
 (segment (start 114.7125 84.0875) (end 116.14 82.66) (width 0.3) (layer "B.Cu") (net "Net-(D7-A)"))
 (segment (start 114.7125 89) (end 114.7125 84.0875) (width 0.3) (layer "B.Cu") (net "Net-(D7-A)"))
 (segment (start 116.14 82.66) (end 119.75 82.66) (width 0.3) (layer "B.Cu") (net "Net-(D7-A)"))
 (segment (start 93.025 86.54) (end 85.26 86.54) (width 0.3) (layer "F.Cu") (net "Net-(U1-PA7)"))
 (segment (start 95.8 89.4) (end 95.8 88) (width 0.3) (layer "F.Cu") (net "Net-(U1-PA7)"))
 (segment (start 85.26 86.54) (end 82.8 89) (width 0.3) (layer "F.Cu") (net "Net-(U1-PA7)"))
 (segment (start 95.8 88) (end 94.34 86.54) (width 0.3) (layer "F.Cu") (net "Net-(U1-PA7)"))
 (segment (start 103 95) (end 101.4 95) (width 0.3) (layer "F.Cu") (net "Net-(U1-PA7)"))
 (segment (start 94.34 86.54) (end 93.025 86.54) (width 0.3) (layer "F.Cu") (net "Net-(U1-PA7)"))
 (segment (start 79.8 89) (end 82.8 89) (width 0.3) (layer "F.Cu") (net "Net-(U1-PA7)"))
 (segment (start 101.4 95) (end 95.8 89.4) (width 0.3) (layer "F.Cu") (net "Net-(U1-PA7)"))
 (segment (start 105.2 97.2) (end 103 95) (width 0.3) (layer "F.Cu") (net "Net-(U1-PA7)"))
 (via (at 79.8 89) (size 0.6) (drill 0.3) (layers "F.Cu" "B.Cu") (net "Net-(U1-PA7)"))
 (segment (start 76.7125 89) (end 79.8 89) (width 0.3) (layer "B.Cu") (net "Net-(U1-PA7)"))
 (segment (start 106.49047 98.49047) (end 110.631618 102.631618) (width 0.3) (layer "F.Cu") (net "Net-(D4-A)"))
 (segment (start 110.631618 102.631618) (end 110.631618 102.72372) (width 0.3) (layer "F.Cu") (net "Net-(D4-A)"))
 (segment (start 106.49047 98.582572) (end 106.49047 98.49047) (width 0.3) (layer "B.Cu") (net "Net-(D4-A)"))
 (segment (start 96.4 99.4) (end 93.025 96.025) (width 0.3) (layer "F.Cu") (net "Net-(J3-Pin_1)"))
 (segment (start 86.99 87.81) (end 93.025 87.81) (width 0.3) (layer "F.Cu") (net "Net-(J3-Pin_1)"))
 (segment (start 80 94.4) (end 80.4 94.4) (width 0.3) (layer "F.Cu") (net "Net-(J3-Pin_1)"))
 (segment (start 80.4 94.4) (end 86.99 87.81) (width 0.3) (layer "F.Cu") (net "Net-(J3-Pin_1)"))
 (segment (start 93.025 96.025) (end 93.025 87.81) (width 0.3) (layer "F.Cu") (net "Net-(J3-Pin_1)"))
 (via (at 96.4 99.4) (size 0.6) (drill 0.3) (layers "F.Cu" "B.Cu") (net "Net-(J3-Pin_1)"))
 (segment (start 96.4 99.4) (end 96.4 101.4875) (width 0.3) (layer "B.Cu") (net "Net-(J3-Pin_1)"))
 (segment (start 75.276279 99.123721) (end 75.276279 99.131618) (width 0.3) (layer "F.Cu") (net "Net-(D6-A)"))
 (segment (start 78.70953 95.69047) (end 75.276279 99.123721) (width 0.3) (layer "F.Cu") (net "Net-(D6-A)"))
 (segment (start 94.2 58.06) (end 94.21 58.05) (width 0.3) (layer "B.Cu") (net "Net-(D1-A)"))
 (segment (start 94.2 62.8875) (end 94.2 58.06) (width 0.3) (layer "B.Cu") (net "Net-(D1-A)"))
 (segment (start 93.025 80.19) (end 94.6 78.615) (width 0.3) (layer "F.Cu") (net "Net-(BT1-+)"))
 (segment (start 94.6 78.615) (end 94.6 77.8) (width 0.3) (layer "F.Cu") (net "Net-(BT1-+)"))
 (segment (start 93.025 85.27) (end 91.52 85.27) (width 0.3) (layer "F.Cu") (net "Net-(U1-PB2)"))
 (segment (start 90.909571 72.445235) (end 108.642265 72.445235) (width 0.3) (layer "F.Cu") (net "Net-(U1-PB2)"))
 (segment (start 89.986961 73.367845) (end 90.909571 72.445235) (width 0.3) (layer "F.Cu") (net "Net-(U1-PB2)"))
 (segment (start 89.986961 83.736961) (end 90 83.75) (width 0.3) (layer "F.Cu") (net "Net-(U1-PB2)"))
 (segment (start 91.52 85.27) (end 90 83.75) (width 0.3) (layer "F.Cu") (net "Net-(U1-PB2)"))
 (segment (start 90 73.380884) (end 89.986961 73.367845) (width 0.3) (layer "F.Cu") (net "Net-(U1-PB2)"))
 (segment (start 90 83.75) (end 90 73.380884) (width 0.3) (layer "F.Cu") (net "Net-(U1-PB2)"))
 (via (at 94.2 72.4) (size 0.6) (drill 0.3) (layers "F.Cu" "B.Cu") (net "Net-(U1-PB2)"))
 (segment (start 94.2 64.7125) (end 94.2 72.4) (width 0.3) (layer "B.Cu") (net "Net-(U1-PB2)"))
 (segment (start 97.41 87.81) (end 95.6 86) (width 0.3) (layer "F.Cu") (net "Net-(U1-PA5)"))
 (segment (start 95.6 86) (end 95.6 85) (width 0.3) (layer "F.Cu") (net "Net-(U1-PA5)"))
 (segment (start 97.975 87.81) (end 97.41 87.81) (width 0.3) (layer "F.Cu") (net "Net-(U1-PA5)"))
 (segment (start 83.645235 68.445235) (end 83.645235 73.154765) (width 0.3) (layer "F.Cu") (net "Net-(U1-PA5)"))
 (via (at 83.6 73.2) (size 0.6) (drill 0.3) (layers "F.Cu" "B.Cu") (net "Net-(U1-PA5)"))
 (via (at 95.6 85) (size 0.6) (drill 0.3) (layers "F.Cu" "B.Cu") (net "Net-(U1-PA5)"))
 (segment (start 83.645235 73.245235) (end 95.4 85) (width 0.3) (layer "B.Cu") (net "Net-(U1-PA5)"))
 (segment (start 95.4 85) (end 95.6 85) (width 0.3) (layer "B.Cu") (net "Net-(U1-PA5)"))
 (segment (start 105.8 89) (end 101.8 85) (width 0.3) (layer "B.Cu") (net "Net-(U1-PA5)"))
 (segment (start 101.8 85) (end 95.6 85) (width 0.3) (layer "B.Cu") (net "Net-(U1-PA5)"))
 (segment (start 112.8875 89) (end 105.8 89) (width 0.3) (layer "B.Cu") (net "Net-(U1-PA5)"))
 (segment (start 78.976279 63.776279) (end 78.868381 63.776279) (width 0.3) (layer "F.Cu") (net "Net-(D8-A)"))
 (segment (start 82.354765 67.154765) (end 78.976279 63.776279) (width 0.3) (layer "F.Cu") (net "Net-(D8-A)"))
 (segment (start 78.976279 63.776279) (end 78.868381 63.776279) (width 0.3) (layer "B.Cu") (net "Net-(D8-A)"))
 (segment (start 96.4 103.3125) (end 96.4 104.2) (width 0.3) (layer "B.Cu") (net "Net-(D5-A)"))
 (segment (start 96.4 104.4) (end 96.4 108.4) (width 0.3) (layer "B.Cu") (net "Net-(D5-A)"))
 (segment (start 69.75 83.59) (end 69.75 86.15) (width 0.3) (layer "B.Cu") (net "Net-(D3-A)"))
 (segment (start 72.6 89) (end 74.8875 89) (width 0.3) (layer "B.Cu") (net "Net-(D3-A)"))
 (segment (start 69.75 86.15) (end 72.6 89) (width 0.3) (layer "B.Cu") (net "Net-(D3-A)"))
 (segment (start 109.932735 71.154765) (end 113.719119 67.368381) (width 0.3) (layer "F.Cu") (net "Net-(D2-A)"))
 (segment (start 113.719119 67.368381) (end 114.22372 67.368381) (width 0.3) (layer "F.Cu") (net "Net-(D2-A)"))
 (segment (start 113.719119 67.368381) (end 114.22372 67.368381) (width 0.3) (layer "B.Cu") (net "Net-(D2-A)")))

